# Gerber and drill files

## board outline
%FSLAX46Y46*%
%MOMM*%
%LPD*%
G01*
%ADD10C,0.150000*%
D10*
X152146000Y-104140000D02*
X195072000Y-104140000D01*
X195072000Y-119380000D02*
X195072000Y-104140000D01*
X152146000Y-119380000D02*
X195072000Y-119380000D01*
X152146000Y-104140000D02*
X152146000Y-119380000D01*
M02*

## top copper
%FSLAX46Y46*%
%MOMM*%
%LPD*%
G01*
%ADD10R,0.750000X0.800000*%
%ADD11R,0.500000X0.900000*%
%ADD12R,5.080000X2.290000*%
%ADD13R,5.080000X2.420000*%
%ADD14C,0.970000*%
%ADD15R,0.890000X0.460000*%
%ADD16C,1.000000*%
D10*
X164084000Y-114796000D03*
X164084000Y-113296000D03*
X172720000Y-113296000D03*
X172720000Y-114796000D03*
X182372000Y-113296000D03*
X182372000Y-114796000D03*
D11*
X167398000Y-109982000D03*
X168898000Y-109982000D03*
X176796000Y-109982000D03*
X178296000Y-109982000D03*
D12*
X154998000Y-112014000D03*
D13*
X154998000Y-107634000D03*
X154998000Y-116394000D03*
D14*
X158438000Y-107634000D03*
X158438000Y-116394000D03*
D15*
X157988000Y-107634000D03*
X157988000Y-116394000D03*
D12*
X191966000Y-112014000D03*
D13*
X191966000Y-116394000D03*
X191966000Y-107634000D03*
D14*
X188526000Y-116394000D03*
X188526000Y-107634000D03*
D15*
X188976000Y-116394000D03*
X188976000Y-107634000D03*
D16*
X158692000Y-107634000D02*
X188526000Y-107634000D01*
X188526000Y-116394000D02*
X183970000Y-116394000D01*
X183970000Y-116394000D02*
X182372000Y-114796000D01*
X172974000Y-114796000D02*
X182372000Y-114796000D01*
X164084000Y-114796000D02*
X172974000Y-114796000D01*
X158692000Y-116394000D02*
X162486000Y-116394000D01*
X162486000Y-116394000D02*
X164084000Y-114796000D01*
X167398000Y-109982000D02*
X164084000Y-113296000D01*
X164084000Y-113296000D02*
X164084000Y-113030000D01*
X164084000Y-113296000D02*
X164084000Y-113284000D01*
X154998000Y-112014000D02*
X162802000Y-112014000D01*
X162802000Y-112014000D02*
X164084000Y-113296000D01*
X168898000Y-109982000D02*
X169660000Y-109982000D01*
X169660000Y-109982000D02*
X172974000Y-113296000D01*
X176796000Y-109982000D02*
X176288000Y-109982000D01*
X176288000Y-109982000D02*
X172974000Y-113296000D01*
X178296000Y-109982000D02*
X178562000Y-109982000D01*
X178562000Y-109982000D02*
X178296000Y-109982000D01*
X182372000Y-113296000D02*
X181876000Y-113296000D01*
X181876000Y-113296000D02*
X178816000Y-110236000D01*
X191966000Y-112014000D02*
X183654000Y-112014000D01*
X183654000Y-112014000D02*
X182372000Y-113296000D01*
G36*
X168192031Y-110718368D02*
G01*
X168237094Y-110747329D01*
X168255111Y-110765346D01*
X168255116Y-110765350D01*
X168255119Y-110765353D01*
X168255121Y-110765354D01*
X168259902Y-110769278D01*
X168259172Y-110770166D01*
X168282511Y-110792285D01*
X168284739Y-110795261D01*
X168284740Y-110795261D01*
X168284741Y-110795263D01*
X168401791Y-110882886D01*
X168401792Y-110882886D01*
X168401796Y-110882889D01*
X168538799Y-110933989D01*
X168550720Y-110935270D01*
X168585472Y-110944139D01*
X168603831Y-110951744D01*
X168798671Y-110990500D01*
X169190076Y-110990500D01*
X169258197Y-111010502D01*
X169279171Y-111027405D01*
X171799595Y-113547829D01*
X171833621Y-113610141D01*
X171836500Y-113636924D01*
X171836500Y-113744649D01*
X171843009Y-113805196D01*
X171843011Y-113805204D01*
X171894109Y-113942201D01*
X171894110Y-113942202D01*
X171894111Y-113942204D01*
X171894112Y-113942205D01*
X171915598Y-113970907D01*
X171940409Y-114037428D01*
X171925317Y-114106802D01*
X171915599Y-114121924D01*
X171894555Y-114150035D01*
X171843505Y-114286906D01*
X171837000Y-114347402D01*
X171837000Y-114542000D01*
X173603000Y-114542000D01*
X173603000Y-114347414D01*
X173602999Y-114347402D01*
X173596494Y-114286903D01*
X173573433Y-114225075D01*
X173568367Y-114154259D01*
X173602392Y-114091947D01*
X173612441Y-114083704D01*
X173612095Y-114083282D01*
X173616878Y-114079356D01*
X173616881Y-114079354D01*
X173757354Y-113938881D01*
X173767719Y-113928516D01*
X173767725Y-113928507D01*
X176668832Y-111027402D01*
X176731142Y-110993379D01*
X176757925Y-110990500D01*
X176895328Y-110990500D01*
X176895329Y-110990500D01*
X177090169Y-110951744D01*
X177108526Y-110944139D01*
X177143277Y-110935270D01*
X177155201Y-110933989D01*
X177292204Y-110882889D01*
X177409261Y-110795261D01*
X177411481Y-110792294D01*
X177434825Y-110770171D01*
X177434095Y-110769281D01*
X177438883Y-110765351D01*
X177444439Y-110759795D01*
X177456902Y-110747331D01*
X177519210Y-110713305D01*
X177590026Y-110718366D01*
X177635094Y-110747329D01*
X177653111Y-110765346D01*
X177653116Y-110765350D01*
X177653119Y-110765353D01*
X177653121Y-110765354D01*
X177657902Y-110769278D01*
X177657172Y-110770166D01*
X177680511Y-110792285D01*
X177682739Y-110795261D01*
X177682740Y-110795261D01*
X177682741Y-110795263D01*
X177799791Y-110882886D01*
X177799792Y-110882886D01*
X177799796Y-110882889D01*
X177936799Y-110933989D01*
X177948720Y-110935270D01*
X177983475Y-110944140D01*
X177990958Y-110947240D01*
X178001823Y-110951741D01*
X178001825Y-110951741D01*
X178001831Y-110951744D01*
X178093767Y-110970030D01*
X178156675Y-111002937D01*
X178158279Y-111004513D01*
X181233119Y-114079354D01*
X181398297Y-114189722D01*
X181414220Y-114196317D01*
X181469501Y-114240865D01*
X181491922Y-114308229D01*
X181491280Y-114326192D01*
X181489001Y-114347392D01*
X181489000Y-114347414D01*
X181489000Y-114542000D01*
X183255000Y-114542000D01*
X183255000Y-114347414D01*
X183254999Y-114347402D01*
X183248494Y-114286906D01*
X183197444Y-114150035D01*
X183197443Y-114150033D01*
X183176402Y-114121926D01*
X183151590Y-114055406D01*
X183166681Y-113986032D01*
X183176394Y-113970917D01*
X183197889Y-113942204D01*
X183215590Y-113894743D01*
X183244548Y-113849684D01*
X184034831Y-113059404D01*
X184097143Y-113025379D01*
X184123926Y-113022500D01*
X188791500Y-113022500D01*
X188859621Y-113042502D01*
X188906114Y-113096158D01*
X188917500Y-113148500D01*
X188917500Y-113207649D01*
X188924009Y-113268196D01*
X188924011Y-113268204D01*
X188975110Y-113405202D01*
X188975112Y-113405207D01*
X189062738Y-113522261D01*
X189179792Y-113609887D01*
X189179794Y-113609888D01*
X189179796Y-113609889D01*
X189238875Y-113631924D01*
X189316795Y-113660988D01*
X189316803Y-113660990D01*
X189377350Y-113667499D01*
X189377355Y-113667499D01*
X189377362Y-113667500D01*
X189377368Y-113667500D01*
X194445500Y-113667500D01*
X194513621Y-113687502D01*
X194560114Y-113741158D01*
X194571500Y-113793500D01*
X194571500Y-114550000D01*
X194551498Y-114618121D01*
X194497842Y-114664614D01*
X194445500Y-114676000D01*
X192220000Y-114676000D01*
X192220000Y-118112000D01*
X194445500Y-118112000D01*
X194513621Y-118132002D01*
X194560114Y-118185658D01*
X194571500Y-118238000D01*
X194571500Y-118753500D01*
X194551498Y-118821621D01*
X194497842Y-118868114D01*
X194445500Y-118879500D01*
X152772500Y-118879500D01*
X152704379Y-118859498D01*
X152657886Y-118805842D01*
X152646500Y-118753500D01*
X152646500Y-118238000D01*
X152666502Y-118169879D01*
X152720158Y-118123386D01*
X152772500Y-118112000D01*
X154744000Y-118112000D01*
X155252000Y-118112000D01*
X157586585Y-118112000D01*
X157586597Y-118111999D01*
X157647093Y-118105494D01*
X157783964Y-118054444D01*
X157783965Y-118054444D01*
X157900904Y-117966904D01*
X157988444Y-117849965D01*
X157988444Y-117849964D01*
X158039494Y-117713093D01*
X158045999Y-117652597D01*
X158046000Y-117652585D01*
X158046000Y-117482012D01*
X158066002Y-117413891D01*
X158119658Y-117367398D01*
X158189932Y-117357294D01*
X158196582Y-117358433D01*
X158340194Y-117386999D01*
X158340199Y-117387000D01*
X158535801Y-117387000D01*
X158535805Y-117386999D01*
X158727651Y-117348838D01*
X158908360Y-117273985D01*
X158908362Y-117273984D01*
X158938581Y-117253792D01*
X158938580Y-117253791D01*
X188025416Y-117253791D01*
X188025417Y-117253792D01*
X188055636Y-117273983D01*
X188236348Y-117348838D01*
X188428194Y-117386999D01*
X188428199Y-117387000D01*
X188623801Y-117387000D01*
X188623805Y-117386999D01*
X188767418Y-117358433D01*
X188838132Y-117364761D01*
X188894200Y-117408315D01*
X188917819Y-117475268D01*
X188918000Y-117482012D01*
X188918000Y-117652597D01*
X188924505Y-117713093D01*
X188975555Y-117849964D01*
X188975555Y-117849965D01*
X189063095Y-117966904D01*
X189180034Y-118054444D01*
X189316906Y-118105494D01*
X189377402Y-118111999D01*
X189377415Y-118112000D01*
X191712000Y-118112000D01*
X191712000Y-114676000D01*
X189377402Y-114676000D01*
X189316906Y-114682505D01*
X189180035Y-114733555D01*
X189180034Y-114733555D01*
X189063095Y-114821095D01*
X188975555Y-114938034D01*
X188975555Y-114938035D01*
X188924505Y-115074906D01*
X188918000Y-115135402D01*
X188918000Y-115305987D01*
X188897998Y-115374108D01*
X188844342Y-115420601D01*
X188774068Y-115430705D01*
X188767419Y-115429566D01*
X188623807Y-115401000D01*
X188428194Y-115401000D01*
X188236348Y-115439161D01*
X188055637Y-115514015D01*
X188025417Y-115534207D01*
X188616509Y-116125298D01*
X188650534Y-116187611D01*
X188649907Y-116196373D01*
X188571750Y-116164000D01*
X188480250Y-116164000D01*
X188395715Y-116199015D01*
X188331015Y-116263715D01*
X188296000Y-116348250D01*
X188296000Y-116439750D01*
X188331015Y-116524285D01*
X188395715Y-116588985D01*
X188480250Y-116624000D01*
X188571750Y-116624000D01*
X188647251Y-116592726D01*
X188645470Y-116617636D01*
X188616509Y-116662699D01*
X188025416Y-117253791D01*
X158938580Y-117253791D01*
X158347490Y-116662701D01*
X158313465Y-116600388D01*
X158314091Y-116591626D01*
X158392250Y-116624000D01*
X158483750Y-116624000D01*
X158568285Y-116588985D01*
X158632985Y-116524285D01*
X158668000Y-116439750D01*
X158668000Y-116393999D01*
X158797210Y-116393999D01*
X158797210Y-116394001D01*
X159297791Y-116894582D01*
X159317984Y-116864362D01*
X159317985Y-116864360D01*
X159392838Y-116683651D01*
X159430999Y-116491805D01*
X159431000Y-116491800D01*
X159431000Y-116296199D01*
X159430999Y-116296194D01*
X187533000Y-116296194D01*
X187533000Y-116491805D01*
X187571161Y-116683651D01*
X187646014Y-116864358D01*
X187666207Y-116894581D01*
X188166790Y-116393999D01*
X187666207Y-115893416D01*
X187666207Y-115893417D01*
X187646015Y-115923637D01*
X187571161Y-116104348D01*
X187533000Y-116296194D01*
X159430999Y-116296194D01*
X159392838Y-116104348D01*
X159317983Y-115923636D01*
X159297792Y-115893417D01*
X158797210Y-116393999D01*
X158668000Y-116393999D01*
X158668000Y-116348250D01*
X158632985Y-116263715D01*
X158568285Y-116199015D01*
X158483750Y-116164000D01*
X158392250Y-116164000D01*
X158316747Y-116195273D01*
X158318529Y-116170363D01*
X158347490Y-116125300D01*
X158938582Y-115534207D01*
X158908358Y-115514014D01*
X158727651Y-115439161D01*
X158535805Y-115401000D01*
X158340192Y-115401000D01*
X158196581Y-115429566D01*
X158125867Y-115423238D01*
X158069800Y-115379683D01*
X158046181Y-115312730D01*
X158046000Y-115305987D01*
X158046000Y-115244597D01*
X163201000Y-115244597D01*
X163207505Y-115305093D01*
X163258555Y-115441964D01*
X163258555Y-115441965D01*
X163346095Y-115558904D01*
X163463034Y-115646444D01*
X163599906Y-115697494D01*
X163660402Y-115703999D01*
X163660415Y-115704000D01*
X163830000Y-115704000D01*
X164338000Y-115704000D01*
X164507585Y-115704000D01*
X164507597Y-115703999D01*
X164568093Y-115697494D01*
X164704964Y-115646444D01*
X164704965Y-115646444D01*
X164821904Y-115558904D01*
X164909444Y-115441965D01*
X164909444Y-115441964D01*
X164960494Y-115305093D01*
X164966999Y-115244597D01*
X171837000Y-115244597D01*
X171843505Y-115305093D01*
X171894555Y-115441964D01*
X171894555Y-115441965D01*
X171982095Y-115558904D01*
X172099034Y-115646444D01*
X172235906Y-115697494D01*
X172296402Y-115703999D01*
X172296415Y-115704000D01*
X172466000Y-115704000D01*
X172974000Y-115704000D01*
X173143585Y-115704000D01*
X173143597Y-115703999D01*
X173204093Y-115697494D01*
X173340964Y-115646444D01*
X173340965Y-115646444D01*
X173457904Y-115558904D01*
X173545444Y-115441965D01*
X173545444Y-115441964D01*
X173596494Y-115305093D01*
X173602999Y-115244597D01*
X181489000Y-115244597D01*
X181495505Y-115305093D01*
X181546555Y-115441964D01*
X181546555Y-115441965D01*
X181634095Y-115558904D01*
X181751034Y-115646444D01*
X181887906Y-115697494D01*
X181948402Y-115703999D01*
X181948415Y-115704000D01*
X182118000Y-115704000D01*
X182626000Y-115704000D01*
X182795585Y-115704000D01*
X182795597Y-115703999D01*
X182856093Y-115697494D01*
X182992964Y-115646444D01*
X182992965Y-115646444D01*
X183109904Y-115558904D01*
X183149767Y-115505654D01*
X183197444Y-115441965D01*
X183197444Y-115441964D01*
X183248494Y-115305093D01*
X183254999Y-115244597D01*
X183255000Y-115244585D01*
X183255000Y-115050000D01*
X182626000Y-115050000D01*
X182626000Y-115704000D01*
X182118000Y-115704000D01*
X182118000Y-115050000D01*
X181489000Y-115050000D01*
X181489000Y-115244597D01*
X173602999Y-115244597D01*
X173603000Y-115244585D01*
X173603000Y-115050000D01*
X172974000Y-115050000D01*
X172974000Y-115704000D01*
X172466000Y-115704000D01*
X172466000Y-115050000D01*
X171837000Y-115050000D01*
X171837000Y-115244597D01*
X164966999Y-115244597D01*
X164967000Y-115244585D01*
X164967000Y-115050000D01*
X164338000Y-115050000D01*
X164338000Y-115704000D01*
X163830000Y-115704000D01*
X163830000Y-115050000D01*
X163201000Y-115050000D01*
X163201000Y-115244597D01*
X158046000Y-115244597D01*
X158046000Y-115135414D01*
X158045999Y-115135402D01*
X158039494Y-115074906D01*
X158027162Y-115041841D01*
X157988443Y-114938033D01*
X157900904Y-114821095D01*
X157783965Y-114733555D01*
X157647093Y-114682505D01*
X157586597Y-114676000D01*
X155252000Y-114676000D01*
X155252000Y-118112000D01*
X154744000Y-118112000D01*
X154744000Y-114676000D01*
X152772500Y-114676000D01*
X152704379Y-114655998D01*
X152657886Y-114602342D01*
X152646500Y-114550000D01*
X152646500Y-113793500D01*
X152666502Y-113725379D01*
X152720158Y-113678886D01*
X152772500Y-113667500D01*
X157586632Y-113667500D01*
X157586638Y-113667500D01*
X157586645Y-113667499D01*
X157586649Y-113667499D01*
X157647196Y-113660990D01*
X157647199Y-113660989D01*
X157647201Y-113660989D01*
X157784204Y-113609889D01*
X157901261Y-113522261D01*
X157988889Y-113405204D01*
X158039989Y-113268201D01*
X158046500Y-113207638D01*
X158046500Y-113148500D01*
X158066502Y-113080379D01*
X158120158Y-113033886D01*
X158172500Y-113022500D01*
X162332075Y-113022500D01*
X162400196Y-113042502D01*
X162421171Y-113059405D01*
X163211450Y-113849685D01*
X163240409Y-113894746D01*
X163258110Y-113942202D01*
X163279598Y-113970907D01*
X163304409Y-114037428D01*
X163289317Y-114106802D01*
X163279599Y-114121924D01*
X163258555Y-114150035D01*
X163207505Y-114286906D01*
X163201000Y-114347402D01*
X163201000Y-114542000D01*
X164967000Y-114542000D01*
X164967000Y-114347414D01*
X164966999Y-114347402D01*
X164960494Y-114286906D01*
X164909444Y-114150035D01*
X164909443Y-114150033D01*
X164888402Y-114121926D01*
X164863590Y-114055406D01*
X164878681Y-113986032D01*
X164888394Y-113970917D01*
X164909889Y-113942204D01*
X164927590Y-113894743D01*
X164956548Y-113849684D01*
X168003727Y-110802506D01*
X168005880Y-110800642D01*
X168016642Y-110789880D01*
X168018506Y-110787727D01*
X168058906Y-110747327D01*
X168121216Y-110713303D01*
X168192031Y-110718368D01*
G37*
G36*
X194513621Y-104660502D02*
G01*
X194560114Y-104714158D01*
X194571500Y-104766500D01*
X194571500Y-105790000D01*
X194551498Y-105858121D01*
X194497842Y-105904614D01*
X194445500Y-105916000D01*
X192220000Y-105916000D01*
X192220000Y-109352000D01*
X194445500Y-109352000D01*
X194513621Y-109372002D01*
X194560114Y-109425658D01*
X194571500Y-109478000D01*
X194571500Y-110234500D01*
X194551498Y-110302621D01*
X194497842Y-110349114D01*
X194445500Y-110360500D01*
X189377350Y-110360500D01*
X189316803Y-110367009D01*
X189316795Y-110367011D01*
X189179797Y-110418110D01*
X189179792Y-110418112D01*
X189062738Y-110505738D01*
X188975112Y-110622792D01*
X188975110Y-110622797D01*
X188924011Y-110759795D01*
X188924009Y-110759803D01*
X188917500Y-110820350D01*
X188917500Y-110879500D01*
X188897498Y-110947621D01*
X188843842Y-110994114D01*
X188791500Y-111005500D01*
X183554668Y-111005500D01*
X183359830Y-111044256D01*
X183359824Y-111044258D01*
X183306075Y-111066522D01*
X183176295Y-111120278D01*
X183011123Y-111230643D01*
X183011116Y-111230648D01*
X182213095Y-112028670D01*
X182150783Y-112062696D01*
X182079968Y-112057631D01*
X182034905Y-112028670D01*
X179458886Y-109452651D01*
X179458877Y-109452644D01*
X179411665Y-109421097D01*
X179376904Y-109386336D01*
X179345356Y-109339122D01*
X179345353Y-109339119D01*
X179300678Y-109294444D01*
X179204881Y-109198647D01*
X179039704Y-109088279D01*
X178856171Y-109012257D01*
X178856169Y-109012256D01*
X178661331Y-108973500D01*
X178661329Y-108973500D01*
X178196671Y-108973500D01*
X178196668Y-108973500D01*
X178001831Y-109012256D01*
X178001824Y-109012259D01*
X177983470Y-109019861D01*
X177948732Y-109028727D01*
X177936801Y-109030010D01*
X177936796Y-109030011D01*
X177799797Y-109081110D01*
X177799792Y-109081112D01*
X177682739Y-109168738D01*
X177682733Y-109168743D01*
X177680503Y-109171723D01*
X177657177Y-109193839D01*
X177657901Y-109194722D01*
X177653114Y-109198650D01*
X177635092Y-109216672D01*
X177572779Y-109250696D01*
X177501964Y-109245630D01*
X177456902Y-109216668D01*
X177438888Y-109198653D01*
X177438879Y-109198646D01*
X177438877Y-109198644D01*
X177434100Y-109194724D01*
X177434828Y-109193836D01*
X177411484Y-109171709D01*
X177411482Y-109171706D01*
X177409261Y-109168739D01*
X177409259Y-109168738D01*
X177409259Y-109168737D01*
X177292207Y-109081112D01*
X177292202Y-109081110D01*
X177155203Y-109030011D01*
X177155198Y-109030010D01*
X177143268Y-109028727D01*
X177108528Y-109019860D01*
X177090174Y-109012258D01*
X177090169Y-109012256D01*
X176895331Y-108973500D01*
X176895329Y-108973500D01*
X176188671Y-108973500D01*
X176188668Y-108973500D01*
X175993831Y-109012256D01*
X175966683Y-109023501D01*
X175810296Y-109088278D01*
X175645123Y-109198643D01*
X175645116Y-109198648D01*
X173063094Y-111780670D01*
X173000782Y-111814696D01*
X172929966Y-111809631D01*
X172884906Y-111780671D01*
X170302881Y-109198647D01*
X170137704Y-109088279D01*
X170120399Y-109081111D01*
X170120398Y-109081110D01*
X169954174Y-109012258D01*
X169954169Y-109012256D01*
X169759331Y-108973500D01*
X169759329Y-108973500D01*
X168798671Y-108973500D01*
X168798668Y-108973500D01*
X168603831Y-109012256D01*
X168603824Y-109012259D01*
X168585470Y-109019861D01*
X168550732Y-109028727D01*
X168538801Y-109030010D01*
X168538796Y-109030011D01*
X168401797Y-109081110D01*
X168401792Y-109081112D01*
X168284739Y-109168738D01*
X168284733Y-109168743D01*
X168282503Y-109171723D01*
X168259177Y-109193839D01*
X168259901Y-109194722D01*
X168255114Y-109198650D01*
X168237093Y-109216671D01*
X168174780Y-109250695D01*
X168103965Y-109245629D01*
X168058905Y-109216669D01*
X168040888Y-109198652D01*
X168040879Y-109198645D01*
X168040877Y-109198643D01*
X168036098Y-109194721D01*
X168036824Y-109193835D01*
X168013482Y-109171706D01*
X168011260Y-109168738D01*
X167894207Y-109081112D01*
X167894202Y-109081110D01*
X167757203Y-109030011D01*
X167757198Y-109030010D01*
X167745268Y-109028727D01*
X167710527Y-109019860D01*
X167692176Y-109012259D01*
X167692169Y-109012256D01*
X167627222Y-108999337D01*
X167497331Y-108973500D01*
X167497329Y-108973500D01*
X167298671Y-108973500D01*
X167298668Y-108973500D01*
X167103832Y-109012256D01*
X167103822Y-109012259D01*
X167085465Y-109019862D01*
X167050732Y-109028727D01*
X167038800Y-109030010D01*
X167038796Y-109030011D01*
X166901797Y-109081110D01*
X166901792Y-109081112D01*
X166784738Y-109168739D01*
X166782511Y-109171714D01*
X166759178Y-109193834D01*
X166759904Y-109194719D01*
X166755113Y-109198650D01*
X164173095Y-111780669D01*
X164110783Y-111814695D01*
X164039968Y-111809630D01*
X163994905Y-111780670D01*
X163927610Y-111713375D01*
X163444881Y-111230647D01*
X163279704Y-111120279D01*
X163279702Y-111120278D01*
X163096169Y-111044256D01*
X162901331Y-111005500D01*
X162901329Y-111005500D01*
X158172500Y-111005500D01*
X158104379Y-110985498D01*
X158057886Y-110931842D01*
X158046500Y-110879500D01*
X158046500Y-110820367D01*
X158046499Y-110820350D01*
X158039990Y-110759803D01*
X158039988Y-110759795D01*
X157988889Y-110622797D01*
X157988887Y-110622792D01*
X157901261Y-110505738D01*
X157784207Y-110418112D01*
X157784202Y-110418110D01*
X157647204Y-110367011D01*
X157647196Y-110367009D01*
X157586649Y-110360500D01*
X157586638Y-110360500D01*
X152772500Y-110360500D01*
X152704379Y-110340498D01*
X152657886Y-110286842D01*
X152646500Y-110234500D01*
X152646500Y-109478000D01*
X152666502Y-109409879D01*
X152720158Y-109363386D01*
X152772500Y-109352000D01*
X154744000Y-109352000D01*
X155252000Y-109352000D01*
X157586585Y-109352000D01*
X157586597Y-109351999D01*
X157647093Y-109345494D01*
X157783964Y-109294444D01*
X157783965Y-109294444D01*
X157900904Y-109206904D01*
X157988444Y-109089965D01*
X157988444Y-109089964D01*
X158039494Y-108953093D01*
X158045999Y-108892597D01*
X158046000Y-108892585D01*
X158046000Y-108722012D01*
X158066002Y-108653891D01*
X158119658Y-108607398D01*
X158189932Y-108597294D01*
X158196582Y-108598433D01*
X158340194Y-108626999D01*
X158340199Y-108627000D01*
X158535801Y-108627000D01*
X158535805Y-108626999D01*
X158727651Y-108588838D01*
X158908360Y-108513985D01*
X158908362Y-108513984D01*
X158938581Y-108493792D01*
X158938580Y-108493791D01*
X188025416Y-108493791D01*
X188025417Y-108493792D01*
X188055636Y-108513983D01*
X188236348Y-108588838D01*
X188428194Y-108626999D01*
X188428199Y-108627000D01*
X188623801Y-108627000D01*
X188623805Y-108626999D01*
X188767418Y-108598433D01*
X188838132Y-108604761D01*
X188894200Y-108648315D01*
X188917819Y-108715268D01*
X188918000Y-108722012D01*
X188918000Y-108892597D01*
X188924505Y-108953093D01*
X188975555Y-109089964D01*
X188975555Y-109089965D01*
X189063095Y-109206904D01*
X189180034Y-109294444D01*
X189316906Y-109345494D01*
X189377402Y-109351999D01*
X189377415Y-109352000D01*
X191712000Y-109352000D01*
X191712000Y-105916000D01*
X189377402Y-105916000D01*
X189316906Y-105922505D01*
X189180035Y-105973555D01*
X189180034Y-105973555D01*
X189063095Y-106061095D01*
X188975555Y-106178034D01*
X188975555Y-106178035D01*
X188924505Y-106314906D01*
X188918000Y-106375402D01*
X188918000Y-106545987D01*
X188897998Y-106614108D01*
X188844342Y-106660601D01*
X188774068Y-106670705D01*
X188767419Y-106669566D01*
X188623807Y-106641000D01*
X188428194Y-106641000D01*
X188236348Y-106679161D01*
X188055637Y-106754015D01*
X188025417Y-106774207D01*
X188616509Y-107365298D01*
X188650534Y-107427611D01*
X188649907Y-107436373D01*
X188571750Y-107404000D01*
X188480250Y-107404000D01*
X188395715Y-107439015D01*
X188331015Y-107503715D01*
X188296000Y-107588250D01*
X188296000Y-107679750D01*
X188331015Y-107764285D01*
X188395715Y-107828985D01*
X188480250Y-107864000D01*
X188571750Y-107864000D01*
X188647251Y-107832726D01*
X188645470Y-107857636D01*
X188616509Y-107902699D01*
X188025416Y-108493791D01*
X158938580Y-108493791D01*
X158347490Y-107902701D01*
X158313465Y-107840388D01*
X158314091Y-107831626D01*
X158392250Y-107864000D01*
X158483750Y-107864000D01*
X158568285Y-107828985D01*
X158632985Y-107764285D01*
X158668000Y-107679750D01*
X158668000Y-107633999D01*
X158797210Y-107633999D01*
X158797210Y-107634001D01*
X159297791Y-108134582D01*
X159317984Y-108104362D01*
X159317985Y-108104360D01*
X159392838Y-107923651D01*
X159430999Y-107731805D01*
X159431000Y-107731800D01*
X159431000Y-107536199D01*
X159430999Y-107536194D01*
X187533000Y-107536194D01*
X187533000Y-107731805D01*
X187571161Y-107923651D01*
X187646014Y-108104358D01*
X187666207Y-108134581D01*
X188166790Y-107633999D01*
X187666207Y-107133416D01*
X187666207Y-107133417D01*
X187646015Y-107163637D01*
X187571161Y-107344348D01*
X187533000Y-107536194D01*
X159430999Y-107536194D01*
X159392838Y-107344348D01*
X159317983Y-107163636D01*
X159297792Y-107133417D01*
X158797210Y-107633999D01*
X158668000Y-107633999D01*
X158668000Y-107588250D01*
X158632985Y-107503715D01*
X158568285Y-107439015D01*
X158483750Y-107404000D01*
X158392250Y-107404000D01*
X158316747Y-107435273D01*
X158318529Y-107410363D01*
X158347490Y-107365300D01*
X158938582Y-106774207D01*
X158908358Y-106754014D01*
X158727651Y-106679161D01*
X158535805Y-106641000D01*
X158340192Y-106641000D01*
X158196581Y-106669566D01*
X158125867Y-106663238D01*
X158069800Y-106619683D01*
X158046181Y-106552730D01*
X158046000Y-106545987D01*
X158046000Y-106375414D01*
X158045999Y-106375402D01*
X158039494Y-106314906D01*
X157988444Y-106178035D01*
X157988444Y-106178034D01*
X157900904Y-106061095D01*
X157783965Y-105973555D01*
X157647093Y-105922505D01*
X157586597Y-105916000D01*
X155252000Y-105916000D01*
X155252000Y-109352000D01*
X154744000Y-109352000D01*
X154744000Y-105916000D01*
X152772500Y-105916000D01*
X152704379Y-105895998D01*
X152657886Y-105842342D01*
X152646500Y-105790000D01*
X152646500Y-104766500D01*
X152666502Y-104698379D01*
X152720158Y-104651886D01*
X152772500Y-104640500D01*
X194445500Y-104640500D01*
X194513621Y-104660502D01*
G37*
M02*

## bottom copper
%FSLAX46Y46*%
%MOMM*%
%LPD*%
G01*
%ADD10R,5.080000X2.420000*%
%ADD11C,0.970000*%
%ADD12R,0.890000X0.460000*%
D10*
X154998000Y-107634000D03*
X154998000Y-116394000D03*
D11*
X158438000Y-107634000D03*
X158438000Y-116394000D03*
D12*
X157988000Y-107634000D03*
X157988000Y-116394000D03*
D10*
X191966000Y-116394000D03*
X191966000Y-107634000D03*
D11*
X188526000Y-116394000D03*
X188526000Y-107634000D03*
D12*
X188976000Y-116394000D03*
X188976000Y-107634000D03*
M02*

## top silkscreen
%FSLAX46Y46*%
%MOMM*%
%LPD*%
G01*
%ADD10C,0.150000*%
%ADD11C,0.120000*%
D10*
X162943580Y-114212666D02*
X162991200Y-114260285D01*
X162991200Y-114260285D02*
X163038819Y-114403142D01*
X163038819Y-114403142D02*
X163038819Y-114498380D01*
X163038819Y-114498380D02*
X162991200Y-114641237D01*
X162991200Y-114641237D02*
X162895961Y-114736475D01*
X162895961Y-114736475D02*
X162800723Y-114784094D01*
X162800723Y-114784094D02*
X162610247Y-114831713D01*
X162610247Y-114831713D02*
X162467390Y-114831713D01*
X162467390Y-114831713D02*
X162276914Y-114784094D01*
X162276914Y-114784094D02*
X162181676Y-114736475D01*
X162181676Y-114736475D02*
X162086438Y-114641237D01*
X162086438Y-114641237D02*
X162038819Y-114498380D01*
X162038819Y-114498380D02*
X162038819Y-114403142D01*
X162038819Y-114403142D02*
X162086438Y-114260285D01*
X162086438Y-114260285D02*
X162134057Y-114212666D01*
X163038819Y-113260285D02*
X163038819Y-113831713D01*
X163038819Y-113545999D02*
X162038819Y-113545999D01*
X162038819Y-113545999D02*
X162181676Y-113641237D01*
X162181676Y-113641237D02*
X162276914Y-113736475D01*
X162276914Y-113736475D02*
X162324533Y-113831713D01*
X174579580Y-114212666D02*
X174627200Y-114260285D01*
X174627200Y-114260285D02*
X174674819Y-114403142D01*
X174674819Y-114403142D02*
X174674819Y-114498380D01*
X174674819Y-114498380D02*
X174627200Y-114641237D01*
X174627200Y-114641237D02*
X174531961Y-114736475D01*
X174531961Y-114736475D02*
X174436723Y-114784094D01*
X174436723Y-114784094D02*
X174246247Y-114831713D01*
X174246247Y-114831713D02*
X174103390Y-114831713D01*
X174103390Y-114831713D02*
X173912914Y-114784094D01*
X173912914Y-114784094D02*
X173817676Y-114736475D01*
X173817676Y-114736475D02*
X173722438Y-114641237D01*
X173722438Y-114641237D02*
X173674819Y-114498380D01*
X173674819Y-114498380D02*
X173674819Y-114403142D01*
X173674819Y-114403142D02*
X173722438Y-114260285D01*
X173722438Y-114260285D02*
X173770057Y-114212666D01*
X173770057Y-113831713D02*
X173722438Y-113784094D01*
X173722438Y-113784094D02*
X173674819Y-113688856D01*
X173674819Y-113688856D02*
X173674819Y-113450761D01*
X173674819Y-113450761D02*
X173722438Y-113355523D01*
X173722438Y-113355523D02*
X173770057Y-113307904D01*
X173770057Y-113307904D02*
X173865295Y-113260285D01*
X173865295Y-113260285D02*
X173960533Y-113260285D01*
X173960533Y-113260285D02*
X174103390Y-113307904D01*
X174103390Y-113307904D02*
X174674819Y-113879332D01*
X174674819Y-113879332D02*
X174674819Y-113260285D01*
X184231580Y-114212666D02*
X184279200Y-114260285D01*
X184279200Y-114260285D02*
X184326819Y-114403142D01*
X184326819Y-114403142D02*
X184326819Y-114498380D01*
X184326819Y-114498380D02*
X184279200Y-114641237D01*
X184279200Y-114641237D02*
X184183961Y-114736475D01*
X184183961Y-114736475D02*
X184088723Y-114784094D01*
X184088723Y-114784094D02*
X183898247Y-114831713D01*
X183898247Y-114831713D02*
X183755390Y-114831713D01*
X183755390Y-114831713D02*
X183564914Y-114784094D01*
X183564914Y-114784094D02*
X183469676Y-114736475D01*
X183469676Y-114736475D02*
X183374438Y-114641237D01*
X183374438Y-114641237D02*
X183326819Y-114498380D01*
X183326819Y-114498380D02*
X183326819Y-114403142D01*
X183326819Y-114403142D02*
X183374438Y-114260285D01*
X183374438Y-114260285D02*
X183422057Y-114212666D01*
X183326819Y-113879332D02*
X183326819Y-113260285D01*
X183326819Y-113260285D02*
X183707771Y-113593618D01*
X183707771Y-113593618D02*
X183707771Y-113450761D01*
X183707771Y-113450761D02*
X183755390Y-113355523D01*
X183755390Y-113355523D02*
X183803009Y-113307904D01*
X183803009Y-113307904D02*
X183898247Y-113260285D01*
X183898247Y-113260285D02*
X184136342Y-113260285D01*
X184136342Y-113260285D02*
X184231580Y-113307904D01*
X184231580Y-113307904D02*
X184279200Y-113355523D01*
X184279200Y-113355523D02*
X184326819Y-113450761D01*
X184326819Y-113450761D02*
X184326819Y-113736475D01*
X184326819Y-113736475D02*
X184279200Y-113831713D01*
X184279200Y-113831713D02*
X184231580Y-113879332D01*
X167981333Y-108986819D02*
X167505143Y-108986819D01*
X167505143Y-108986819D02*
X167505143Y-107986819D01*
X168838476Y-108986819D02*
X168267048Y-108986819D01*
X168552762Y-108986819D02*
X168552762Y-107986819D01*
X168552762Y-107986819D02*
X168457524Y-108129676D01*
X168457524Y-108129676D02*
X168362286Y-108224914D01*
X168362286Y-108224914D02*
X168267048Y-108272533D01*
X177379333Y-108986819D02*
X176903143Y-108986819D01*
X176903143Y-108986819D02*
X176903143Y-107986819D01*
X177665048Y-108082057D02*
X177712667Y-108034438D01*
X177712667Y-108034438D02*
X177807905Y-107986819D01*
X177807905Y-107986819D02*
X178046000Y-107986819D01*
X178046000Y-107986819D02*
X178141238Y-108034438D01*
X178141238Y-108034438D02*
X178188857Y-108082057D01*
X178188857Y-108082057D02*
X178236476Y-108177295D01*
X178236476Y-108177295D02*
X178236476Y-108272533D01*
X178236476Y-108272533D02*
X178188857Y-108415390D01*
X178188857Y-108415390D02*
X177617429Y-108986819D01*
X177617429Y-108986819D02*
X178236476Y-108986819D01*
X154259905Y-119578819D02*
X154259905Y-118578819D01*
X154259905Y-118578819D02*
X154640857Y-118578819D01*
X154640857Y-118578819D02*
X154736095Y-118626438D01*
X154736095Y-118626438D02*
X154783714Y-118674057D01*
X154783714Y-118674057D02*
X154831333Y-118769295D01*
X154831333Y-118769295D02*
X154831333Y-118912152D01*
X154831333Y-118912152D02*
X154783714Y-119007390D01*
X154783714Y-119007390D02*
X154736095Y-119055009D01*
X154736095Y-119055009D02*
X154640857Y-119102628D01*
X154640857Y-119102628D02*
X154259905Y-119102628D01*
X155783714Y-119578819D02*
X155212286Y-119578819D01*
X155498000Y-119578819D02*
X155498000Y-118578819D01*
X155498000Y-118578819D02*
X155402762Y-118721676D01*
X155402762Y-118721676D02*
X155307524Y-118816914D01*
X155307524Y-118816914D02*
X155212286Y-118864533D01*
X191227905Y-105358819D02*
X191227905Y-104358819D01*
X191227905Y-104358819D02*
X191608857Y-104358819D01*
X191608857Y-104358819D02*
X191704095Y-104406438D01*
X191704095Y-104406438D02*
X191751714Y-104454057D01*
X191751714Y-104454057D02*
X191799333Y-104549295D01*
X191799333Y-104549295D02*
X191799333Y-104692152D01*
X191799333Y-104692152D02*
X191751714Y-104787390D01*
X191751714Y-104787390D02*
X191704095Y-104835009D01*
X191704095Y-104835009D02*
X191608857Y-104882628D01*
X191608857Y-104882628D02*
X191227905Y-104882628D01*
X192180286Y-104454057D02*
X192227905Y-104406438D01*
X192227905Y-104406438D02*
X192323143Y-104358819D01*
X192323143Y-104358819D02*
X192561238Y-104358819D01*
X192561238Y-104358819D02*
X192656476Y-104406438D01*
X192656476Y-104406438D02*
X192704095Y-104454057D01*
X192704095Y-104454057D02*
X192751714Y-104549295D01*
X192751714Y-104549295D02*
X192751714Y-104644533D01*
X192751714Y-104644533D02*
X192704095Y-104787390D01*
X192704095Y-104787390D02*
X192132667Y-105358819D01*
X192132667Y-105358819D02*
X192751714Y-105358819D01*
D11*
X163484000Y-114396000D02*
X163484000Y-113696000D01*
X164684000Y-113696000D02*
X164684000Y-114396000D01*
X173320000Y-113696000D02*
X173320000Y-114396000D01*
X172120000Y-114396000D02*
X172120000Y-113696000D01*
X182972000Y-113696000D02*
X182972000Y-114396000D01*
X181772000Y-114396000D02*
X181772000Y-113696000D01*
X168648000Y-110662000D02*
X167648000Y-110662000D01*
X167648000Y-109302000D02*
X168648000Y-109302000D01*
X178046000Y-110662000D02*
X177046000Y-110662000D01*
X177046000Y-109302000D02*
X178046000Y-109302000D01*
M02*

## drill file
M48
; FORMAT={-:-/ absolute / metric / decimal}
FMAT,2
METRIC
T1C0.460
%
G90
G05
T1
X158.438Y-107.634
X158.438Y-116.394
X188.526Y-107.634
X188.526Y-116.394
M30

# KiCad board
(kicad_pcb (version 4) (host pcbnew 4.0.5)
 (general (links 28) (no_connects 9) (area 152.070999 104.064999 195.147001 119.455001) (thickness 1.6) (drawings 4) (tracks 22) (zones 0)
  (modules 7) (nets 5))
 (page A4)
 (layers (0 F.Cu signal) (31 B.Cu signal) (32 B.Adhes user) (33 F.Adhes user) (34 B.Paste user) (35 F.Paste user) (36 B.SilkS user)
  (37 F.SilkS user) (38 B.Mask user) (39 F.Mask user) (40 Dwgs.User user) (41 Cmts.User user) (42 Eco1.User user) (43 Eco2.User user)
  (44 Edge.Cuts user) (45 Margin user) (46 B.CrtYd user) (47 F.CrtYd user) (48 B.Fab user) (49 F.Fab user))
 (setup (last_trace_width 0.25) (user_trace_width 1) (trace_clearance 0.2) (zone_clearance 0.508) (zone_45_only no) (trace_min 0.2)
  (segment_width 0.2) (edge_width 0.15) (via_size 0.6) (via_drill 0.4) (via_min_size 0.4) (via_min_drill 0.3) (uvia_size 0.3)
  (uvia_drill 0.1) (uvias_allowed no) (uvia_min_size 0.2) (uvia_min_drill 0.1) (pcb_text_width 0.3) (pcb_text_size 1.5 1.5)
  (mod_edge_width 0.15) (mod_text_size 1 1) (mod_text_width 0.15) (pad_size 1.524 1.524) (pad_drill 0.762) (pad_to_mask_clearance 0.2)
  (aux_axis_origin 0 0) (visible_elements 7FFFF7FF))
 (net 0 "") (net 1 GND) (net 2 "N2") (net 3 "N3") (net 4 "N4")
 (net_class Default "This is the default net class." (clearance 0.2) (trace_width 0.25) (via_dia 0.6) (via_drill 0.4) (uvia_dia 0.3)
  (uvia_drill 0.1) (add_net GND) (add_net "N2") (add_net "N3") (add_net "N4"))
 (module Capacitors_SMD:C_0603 (layer F.Cu) (at 164.084 114.046 90)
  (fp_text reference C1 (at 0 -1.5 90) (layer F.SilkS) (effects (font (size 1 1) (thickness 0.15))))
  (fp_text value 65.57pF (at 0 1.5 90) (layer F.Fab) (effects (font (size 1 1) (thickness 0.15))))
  (fp_line (start -0.35 -0.6) (end 0.35 -0.6) (layer F.SilkS) (width 0.12))
  (fp_line (start 0.35 0.6) (end -0.35 0.6) (layer F.SilkS) (width 0.12))
  (pad 1 smd rect (at -0.75 0 90) (size 0.8 0.75) (layers F.Cu F.Paste F.Mask) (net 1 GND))
  (pad 2 smd rect (at 0.75 0 90) (size 0.8 0.75) (layers F.Cu F.Paste F.Mask) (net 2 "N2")))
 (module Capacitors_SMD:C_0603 (layer F.Cu) (at 172.72 114.046 270)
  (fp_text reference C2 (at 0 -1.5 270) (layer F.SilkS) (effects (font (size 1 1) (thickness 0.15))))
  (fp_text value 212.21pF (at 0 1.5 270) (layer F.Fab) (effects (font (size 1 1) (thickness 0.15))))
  (fp_line (start -0.35 -0.6) (end 0.35 -0.6) (layer F.SilkS) (width 0.12))
  (fp_line (start 0.35 0.6) (end -0.35 0.6) (layer F.SilkS) (width 0.12))
  (pad 1 smd rect (at -0.75 0 270) (size 0.8 0.75) (layers F.Cu F.Paste F.Mask) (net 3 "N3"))
  (pad 2 smd rect (at 0.75 0 270) (size 0.8 0.75) (layers F.Cu F.Paste F.Mask) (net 1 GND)))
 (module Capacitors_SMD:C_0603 (layer F.Cu) (at 182.372 114.046 270)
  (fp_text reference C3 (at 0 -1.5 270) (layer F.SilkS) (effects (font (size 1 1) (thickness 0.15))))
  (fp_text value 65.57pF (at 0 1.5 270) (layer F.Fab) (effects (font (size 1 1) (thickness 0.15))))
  (fp_line (start -0.35 -0.6) (end 0.35 -0.6) (layer F.SilkS) (width 0.12))
  (fp_line (start 0.35 0.6) (end -0.35 0.6) (layer F.SilkS) (width 0.12))
  (pad 1 smd rect (at -0.75 0 270) (size 0.8 0.75) (layers F.Cu F.Paste F.Mask) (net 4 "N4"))
  (pad 2 smd rect (at 0.75 0 270) (size 0.8 0.75) (layers F.Cu F.Paste F.Mask) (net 1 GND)))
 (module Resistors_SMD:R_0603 (layer F.Cu) (at 168.148 109.982)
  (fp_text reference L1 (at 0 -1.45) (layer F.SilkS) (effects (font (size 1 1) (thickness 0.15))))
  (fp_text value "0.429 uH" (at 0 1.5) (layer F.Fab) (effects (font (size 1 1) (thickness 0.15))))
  (fp_line (start 0.5 0.68) (end -0.5 0.68) (layer F.SilkS) (width 0.12))
  (fp_line (start -0.5 -0.68) (end 0.5 -0.68) (layer F.SilkS) (width 0.12))
  (pad 1 smd rect (at -0.75 0) (size 0.5 0.9) (layers F.Cu F.Paste F.Mask) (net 2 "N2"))
  (pad 2 smd rect (at 0.75 0) (size 0.5 0.9) (layers F.Cu F.Paste F.Mask) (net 3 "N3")))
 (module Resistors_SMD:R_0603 (layer F.Cu) (at 177.546 109.982)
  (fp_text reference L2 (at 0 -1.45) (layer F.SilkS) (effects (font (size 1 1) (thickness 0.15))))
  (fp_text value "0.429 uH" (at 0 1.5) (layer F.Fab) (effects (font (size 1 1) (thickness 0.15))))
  (fp_line (start 0.5 0.68) (end -0.5 0.68) (layer F.SilkS) (width 0.12))
  (fp_line (start -0.5 -0.68) (end 0.5 -0.68) (layer F.SilkS) (width 0.12))
  (pad 1 smd rect (at -0.75 0) (size 0.5 0.9) (layers F.Cu F.Paste F.Mask) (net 3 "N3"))
  (pad 2 smd rect (at 0.75 0) (size 0.5 0.9) (layers F.Cu F.Paste F.Mask) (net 4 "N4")))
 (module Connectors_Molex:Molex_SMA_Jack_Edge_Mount (layer F.Cu) (at 156.718 112.014)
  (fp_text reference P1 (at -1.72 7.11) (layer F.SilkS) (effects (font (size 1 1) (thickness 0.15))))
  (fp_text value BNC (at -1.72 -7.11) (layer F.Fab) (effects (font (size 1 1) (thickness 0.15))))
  (pad 1 smd rect (at -1.72 0) (size 5.08 2.29) (layers F.Cu F.Paste F.Mask) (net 2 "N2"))
  (pad 2 smd rect (at -1.72 -4.38) (size 5.08 2.42) (layers F.Cu F.Paste F.Mask) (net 1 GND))
  (pad 2 smd rect (at -1.72 4.38) (size 5.08 2.42) (layers F.Cu F.Paste F.Mask) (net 1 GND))
  (pad 2 smd rect (at -1.72 -4.38) (size 5.08 2.42) (layers B.Cu B.Paste B.Mask) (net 1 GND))
  (pad 2 smd rect (at -1.72 4.38) (size 5.08 2.42) (layers B.Cu B.Paste B.Mask) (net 1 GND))
  (pad 2 thru_hole circle (at 1.72 -4.38) (size 0.97 0.97) (drill 0.46) (layers *.Cu) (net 1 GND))
  (pad 2 thru_hole circle (at 1.72 4.38) (size 0.97 0.97) (drill 0.46) (layers *.Cu) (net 1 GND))
  (pad 2 smd rect (at 1.27 -4.38) (size 0.89 0.46) (layers F.Cu) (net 1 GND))
  (pad 2 smd rect (at 1.27 4.38) (size 0.89 0.46) (layers F.Cu) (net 1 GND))
  (pad 2 smd rect (at 1.27 -4.38) (size 0.89 0.46) (layers B.Cu) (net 1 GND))
  (pad 2 smd rect (at 1.27 4.38) (size 0.89 0.46) (layers B.Cu) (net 1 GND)))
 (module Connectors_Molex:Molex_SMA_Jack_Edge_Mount (layer F.Cu) (at 190.246 112.014 180)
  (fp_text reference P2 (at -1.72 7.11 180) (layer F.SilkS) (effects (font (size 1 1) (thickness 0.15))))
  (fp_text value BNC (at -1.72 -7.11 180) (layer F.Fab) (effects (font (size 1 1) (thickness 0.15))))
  (pad 1 smd rect (at -1.72 0 180) (size 5.08 2.29) (layers F.Cu F.Paste F.Mask) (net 4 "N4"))
  (pad 2 smd rect (at -1.72 -4.38 180) (size 5.08 2.42) (layers F.Cu F.Paste F.Mask) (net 1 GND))
  (pad 2 smd rect (at -1.72 4.38 180) (size 5.08 2.42) (layers F.Cu F.Paste F.Mask) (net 1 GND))
  (pad 2 smd rect (at -1.72 -4.38 180) (size 5.08 2.42) (layers B.Cu B.Paste B.Mask) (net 1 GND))
  (pad 2 smd rect (at -1.72 4.38 180) (size 5.08 2.42) (layers B.Cu B.Paste B.Mask) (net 1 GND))
  (pad 2 thru_hole circle (at 1.72 -4.38 180) (size 0.97 0.97) (drill 0.46) (layers *.Cu) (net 1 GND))
  (pad 2 thru_hole circle (at 1.72 4.38 180) (size 0.97 0.97) (drill 0.46) (layers *.Cu) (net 1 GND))
  (pad 2 smd rect (at 1.27 -4.38 180) (size 0.89 0.46) (layers F.Cu) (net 1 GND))
  (pad 2 smd rect (at 1.27 4.38 180) (size 0.89 0.46) (layers F.Cu) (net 1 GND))
  (pad 2 smd rect (at 1.27 -4.38 180) (size 0.89 0.46) (layers B.Cu) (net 1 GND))
  (pad 2 smd rect (at 1.27 4.38 180) (size 0.89 0.46) (layers B.Cu) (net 1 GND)))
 (gr_line (start 152.146 104.14) (end 195.072 104.14) (layer Edge.Cuts) (width 0.15))
 (gr_line (start 195.072 119.38) (end 195.072 104.14) (layer Edge.Cuts) (width 0.15))
 (gr_line (start 152.146 119.38) (end 195.072 119.38) (layer Edge.Cuts) (width 0.15))
 (gr_line (start 152.146 104.14) (end 152.146 119.38) (layer Edge.Cuts) (width 0.15))
 (segment (start 158.692 107.634) (end 188.526 107.634) (width 1) (layer F.Cu) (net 1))
 (segment (start 188.526 116.394) (end 183.97 116.394) (width 1) (layer F.Cu) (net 1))
 (segment (start 183.97 116.394) (end 182.372 114.796) (width 1) (layer F.Cu) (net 1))
 (segment (start 172.974 114.796) (end 182.372 114.796) (width 1) (layer F.Cu) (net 1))
 (segment (start 164.084 114.796) (end 172.974 114.796) (width 1) (layer F.Cu) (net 1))
 (segment (start 158.692 116.394) (end 162.486 116.394) (width 1) (layer F.Cu) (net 1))
 (segment (start 162.486 116.394) (end 164.084 114.796) (width 1) (layer F.Cu) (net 1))
 (segment (start 167.398 109.982) (end 164.084 113.296) (width 1) (layer F.Cu) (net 2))
 (segment (start 164.084 113.296) (end 164.084 113.03) (width 1) (layer F.Cu) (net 2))
 (segment (start 164.084 113.296) (end 164.084 113.284) (width 1) (layer F.Cu) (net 2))
 (segment (start 154.998 112.014) (end 162.802 112.014) (width 1) (layer F.Cu) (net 2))
 (segment (start 162.802 112.014) (end 164.084 113.296) (width 1) (layer F.Cu) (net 2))
 (segment (start 168.898 109.982) (end 169.66 109.982) (width 1) (layer F.Cu) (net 3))
 (segment (start 169.66 109.982) (end 172.974 113.296) (width 1) (layer F.Cu) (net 3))
 (segment (start 176.796 109.982) (end 176.288 109.982) (width 1) (layer F.Cu) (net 3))
 (segment (start 176.288 109.982) (end 172.974 113.296) (width 1) (layer F.Cu) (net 3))
 (segment (start 178.296 109.982) (end 178.562 109.982) (width 1) (layer F.Cu) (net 4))
 (segment (start 178.562 109.982) (end 178.296 109.982) (width 1) (layer F.Cu) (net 4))
 (segment (start 182.372 113.296) (end 181.876 113.296) (width 1) (layer F.Cu) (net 4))
 (segment (start 181.876 113.296) (end 178.816 110.236) (width 1) (layer F.Cu) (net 4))
 (segment (start 191.966 112.014) (end 183.654 112.014) (width 1) (layer F.Cu) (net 4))
 (segment (start 183.654 112.014) (end 182.372 113.296) (width 1) (layer F.Cu) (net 4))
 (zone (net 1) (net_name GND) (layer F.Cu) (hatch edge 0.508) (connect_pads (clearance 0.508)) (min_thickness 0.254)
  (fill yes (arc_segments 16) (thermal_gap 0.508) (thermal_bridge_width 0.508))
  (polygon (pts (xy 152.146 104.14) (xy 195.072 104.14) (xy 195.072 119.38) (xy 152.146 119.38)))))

